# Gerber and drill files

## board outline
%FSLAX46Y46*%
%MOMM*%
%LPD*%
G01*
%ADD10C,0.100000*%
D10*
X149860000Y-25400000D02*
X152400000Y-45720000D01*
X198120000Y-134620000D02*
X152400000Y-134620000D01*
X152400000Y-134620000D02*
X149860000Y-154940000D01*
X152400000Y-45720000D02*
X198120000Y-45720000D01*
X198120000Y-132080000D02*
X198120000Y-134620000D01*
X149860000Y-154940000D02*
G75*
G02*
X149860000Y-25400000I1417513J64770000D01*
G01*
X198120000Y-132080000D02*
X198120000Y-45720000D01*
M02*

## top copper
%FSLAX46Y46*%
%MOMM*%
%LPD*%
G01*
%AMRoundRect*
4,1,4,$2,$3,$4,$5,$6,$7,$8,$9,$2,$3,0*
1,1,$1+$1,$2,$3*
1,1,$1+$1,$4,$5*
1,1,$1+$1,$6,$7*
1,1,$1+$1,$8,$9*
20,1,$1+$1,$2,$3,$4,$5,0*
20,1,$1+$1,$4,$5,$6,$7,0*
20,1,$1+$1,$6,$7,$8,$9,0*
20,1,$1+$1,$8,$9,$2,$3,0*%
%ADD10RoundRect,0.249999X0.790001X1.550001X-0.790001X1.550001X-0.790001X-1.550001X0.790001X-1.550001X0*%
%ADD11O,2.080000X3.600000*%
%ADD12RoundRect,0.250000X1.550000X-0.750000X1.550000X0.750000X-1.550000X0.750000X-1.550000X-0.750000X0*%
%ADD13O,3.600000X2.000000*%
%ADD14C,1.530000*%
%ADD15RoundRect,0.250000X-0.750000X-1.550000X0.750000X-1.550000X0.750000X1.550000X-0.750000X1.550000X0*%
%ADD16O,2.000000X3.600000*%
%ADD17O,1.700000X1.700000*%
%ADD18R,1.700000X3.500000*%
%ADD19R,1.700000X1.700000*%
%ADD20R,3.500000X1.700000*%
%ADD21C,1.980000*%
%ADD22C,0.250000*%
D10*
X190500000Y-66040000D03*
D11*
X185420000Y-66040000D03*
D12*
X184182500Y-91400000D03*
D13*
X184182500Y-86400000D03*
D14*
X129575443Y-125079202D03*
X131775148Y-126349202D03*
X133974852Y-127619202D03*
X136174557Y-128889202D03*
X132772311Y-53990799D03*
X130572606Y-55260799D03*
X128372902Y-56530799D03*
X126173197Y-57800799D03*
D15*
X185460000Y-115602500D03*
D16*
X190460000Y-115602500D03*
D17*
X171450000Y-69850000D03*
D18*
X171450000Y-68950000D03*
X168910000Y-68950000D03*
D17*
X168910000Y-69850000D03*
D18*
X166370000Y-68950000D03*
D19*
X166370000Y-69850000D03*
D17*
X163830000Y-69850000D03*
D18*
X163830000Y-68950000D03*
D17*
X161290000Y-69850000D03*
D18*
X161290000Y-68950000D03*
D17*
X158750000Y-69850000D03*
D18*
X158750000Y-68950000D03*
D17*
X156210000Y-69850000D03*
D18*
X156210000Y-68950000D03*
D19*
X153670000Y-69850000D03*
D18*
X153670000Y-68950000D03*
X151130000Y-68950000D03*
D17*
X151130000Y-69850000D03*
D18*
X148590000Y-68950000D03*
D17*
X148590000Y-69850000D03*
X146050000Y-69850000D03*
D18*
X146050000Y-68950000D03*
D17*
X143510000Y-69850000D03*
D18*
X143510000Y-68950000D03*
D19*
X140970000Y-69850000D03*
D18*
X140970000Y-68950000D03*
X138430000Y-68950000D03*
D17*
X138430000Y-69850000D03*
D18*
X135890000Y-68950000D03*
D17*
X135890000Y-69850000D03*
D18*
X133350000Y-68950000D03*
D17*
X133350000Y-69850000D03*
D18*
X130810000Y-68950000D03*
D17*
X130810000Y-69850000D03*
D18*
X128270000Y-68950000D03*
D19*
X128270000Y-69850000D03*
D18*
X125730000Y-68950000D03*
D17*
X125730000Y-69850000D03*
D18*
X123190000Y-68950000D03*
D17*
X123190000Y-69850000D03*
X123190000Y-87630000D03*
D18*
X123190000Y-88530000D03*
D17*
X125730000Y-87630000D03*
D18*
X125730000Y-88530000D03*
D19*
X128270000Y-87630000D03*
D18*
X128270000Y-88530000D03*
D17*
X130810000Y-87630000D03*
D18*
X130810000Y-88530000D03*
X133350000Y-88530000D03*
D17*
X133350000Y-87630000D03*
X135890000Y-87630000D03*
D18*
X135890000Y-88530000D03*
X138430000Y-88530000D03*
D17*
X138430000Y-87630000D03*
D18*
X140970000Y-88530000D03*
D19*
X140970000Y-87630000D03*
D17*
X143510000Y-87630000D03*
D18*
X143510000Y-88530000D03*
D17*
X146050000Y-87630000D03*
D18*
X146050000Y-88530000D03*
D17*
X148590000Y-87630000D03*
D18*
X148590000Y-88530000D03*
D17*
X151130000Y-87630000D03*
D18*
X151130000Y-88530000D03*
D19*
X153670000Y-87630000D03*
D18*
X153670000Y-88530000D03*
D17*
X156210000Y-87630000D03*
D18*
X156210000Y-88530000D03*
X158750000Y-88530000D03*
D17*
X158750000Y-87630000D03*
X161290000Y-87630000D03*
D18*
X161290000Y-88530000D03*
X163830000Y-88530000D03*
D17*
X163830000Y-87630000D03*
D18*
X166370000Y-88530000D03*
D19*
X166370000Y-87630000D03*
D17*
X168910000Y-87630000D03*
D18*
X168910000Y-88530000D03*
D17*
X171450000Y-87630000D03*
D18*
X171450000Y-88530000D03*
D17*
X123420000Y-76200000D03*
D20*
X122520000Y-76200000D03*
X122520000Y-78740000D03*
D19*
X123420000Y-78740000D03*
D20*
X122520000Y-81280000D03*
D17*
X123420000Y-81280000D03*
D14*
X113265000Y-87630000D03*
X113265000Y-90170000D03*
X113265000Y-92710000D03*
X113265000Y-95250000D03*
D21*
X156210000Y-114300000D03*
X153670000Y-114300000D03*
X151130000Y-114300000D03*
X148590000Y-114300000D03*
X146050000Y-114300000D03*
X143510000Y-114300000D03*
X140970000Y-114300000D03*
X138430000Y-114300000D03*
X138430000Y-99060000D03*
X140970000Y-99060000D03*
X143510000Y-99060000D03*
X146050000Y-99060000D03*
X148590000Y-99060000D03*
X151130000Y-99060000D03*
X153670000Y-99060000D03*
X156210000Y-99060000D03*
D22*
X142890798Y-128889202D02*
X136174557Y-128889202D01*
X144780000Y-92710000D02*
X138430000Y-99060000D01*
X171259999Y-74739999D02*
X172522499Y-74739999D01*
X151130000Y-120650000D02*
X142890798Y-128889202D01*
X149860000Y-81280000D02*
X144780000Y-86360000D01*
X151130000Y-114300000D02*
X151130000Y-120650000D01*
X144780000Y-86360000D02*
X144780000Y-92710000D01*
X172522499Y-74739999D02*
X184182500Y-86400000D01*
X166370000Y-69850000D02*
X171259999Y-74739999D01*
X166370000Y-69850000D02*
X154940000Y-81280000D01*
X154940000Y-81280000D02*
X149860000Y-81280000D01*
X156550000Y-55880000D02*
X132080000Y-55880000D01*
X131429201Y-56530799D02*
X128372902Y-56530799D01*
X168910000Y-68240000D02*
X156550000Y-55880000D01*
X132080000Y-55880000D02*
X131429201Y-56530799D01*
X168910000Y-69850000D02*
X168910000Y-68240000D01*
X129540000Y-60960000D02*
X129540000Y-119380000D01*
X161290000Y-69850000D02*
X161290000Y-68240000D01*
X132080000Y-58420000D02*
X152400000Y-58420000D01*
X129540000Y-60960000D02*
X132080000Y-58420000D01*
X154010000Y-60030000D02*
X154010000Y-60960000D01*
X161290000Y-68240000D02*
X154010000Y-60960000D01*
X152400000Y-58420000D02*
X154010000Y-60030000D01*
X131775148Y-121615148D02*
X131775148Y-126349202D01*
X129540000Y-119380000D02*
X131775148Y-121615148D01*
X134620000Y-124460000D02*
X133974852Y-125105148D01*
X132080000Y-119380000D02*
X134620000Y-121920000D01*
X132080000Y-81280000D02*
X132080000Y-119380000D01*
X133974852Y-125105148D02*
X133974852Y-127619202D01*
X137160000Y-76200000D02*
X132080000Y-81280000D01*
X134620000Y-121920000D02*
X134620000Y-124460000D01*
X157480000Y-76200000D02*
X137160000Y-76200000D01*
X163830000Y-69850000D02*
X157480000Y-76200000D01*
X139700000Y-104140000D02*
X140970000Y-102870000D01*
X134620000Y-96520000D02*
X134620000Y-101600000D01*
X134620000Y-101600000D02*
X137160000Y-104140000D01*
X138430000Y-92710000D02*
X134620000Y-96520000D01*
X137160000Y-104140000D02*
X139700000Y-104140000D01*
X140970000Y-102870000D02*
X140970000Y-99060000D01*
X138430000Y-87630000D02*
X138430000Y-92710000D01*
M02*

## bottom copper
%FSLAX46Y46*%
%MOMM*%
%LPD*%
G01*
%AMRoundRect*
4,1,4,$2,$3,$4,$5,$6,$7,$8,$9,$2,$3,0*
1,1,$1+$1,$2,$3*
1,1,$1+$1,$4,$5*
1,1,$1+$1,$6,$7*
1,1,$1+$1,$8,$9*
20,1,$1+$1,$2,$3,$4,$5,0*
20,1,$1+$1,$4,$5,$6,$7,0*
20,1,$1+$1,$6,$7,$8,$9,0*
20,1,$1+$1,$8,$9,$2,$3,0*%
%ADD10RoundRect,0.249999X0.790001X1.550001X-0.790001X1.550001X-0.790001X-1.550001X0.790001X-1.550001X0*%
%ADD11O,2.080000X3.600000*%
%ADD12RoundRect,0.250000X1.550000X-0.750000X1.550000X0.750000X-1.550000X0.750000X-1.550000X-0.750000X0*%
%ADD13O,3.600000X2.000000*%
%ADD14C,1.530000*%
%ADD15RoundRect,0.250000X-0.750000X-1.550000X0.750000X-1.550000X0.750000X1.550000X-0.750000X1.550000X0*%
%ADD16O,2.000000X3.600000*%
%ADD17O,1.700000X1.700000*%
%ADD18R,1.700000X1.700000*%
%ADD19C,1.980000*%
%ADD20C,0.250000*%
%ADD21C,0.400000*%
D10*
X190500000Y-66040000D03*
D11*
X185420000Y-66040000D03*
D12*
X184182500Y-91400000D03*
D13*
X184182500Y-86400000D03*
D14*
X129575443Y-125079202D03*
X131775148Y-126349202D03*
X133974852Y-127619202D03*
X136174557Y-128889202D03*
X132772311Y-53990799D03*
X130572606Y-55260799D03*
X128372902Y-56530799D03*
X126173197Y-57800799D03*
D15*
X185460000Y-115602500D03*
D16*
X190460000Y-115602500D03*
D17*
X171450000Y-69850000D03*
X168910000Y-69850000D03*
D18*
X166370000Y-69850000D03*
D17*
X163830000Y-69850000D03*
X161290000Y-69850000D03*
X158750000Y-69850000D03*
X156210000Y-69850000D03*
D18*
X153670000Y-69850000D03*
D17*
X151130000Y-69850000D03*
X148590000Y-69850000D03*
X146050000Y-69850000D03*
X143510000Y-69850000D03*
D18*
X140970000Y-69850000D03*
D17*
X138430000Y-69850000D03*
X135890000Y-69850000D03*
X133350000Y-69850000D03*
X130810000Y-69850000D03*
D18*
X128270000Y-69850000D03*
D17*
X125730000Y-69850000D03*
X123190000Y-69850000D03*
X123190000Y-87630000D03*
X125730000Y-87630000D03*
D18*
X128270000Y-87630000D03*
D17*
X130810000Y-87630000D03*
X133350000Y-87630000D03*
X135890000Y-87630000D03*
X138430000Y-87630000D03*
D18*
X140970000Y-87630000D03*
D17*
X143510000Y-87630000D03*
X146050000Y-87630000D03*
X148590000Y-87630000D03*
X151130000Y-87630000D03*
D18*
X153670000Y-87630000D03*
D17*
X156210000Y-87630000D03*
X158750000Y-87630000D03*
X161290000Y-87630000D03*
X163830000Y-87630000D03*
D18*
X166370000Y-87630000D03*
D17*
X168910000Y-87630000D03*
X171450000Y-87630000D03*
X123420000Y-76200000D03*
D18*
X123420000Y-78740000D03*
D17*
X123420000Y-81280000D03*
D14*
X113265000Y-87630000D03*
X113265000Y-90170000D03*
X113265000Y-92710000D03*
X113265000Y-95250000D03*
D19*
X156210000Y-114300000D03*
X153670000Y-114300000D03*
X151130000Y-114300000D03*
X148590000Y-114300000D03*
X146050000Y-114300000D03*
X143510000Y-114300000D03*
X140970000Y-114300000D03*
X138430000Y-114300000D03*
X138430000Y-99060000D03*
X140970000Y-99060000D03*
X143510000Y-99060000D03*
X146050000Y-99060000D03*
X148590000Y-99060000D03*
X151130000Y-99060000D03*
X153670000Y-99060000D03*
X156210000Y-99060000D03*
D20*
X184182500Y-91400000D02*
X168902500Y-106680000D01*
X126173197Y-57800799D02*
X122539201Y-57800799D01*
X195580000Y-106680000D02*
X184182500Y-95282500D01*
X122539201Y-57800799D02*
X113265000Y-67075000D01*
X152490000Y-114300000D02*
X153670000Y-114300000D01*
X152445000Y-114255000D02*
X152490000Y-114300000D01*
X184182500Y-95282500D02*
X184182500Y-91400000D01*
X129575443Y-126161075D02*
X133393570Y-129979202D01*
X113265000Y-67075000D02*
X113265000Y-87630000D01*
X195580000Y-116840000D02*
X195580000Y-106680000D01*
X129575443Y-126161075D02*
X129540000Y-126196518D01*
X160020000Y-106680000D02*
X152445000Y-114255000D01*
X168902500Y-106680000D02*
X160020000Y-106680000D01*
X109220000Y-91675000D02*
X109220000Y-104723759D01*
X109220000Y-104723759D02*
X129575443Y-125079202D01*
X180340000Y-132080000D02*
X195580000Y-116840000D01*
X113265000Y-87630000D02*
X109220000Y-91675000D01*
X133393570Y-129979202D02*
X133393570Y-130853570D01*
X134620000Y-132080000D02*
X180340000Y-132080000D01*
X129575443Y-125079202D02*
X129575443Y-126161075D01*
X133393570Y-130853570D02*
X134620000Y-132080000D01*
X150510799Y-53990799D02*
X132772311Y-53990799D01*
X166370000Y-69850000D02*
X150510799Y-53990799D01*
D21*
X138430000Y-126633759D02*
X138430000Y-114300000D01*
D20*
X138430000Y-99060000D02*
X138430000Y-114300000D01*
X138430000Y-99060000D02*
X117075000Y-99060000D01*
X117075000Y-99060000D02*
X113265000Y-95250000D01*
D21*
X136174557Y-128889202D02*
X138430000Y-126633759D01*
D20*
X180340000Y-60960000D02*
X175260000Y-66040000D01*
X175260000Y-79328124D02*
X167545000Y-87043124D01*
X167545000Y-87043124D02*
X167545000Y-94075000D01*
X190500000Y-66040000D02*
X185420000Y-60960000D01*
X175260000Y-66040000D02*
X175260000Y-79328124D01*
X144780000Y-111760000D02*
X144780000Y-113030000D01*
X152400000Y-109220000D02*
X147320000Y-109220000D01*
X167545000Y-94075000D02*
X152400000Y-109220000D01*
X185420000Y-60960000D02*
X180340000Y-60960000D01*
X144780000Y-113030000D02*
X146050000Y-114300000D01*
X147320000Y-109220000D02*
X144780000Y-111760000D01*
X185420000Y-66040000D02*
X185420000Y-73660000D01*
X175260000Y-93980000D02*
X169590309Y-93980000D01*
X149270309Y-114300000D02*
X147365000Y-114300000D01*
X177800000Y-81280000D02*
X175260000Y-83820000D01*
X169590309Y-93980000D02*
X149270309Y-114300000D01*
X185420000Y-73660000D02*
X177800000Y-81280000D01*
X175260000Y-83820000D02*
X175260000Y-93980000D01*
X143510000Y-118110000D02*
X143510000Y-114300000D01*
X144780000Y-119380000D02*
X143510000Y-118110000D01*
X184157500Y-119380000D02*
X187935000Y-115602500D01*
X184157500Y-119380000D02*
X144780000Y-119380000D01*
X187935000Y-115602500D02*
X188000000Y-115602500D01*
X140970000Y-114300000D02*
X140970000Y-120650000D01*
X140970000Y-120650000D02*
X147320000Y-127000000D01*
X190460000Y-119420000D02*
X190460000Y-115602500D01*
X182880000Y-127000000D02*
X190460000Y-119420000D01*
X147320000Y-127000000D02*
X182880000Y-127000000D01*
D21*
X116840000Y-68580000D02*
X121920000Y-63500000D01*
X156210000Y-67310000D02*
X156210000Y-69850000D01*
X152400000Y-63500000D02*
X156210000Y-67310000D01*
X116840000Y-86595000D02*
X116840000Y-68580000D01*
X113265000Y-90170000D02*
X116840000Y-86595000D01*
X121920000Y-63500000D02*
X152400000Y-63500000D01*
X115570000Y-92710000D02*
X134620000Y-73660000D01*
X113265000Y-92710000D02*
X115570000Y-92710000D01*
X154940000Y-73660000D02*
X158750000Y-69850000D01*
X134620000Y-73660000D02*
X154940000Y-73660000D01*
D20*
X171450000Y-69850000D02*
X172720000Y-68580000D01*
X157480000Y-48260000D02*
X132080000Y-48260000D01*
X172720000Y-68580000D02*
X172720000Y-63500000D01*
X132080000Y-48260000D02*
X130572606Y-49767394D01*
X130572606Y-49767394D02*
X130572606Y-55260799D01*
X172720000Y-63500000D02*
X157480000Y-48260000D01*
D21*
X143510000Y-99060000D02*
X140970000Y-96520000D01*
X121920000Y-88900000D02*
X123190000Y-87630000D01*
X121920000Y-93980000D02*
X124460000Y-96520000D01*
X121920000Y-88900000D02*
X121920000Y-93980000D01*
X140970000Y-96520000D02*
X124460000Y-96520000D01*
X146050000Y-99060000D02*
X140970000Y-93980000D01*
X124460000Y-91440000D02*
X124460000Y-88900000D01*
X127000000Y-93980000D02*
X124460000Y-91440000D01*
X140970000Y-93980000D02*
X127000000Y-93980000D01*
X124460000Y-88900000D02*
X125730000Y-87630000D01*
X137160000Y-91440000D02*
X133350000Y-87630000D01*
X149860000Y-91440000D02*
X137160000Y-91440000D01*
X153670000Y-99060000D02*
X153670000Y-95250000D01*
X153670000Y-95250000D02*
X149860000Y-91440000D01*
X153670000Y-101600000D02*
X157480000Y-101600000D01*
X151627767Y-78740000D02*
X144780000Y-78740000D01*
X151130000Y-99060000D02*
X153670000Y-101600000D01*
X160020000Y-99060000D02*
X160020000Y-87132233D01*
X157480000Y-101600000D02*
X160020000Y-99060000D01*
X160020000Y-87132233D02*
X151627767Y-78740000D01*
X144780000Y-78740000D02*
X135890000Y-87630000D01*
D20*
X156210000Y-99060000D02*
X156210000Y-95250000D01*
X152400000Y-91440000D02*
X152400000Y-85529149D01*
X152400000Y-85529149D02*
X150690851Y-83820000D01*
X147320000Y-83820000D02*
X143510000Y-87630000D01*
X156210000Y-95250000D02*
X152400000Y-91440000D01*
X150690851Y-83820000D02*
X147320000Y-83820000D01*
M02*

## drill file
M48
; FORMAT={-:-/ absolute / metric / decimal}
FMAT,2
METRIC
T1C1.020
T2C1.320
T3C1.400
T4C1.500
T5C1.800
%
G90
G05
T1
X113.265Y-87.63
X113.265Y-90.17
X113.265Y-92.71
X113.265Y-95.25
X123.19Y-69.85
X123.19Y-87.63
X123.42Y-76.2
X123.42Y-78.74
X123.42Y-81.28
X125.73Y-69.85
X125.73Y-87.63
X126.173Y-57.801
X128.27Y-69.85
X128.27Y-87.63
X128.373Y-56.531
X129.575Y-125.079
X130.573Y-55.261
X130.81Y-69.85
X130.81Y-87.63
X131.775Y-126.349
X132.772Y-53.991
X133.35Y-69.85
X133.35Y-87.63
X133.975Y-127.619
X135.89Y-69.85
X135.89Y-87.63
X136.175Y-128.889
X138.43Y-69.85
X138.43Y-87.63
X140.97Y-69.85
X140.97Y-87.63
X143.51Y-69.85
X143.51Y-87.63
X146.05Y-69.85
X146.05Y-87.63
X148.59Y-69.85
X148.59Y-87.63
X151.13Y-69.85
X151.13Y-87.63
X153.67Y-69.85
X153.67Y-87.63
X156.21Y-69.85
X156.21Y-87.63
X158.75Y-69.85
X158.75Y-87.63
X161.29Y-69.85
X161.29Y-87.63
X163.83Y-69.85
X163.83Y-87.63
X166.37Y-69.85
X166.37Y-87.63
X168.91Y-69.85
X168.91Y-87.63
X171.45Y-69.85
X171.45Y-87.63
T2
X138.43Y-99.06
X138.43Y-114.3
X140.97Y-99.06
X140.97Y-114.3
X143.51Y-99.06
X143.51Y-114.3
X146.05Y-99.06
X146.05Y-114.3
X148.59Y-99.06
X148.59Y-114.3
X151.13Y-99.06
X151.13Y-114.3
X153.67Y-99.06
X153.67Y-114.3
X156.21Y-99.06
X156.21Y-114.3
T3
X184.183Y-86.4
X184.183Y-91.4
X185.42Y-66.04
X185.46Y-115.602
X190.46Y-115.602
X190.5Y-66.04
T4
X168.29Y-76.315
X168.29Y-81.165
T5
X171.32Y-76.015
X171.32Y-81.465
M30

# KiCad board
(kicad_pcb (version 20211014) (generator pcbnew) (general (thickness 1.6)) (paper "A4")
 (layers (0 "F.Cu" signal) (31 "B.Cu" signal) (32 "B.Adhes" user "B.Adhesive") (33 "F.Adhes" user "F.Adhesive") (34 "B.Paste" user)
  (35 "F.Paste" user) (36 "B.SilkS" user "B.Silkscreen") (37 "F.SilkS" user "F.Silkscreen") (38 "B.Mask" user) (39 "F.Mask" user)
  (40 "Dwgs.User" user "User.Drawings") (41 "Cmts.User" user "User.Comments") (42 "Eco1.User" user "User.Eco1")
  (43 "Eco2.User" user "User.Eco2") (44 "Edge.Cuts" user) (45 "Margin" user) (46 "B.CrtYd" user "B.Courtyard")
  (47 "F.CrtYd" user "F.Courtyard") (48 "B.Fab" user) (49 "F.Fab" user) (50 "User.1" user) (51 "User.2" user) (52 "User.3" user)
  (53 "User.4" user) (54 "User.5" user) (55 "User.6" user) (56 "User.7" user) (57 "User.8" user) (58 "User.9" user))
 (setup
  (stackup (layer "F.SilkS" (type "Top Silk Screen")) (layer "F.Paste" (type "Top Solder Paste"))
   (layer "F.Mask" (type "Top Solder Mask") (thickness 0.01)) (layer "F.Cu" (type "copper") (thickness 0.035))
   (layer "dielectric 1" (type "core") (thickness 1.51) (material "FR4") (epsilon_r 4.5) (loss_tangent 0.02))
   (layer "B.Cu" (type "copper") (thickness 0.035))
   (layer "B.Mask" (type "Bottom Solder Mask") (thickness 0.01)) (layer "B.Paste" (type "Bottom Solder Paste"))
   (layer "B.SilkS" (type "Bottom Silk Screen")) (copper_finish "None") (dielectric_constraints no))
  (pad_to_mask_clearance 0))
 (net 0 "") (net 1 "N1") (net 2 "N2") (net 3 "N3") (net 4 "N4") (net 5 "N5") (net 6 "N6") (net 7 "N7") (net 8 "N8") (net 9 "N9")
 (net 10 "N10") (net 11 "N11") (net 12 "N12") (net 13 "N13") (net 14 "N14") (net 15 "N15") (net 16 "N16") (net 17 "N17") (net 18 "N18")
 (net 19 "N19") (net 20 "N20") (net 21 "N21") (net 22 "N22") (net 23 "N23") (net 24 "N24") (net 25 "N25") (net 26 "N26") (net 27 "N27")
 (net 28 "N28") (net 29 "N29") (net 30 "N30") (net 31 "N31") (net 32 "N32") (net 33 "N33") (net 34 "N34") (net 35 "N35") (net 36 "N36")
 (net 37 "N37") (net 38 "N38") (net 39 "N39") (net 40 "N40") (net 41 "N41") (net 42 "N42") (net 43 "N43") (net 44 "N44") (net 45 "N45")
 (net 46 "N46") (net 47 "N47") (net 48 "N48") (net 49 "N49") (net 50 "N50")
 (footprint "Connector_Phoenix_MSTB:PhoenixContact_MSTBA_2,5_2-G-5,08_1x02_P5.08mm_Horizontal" (layer "F.Cu") (at 190.5 66.04 180)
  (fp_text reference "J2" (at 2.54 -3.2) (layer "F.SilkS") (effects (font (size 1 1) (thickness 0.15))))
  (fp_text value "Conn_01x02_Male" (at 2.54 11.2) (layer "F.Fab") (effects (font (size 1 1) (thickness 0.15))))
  (pad "1" thru_hole roundrect (at 0 0 180) (size 2.08 3.6) (drill 1.4) (layers *.Cu *.Mask) (roundrect_rratio 0.120192) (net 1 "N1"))
  (pad "2" thru_hole oval (at 5.08 0 180) (size 2.08 3.6) (drill 1.4) (layers *.Cu *.Mask) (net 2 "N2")))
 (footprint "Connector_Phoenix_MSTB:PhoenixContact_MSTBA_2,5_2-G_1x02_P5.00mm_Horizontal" (layer "F.Cu") (at 184.1825 91.4 90)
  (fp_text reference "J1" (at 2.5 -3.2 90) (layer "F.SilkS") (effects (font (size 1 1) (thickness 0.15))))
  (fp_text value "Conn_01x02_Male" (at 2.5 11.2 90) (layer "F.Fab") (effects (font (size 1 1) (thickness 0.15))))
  (pad "1" thru_hole roundrect (at 0 0 90) (size 2 3.6) (drill 1.4) (layers *.Cu *.Mask) (roundrect_rratio 0.125) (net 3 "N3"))
  (pad "2" thru_hole oval (at 5 0 90) (size 2 3.6) (drill 1.4) (layers *.Cu *.Mask) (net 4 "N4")))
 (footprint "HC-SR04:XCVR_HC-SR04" (layer "F.Cu") (at 132.875 126.984202 -30)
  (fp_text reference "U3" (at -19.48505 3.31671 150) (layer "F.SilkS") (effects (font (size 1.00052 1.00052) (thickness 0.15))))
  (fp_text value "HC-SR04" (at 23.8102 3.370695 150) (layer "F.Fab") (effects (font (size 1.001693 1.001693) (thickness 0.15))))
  (pad "1" thru_hole circle locked (at -3.81 0 330) (size 1.53 1.53) (drill 1.02) (layers *.Cu *.Mask) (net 3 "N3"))
  (pad "2" thru_hole circle locked (at -1.27 0 330) (size 1.53 1.53) (drill 1.02) (layers *.Cu *.Mask) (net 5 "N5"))
  (pad "3" thru_hole circle locked (at 1.27 0 330) (size 1.53 1.53) (drill 1.02) (layers *.Cu *.Mask) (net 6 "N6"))
  (pad "4" thru_hole circle locked (at 3.81 0 330) (size 1.53 1.53) (drill 1.02) (layers *.Cu *.Mask) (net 4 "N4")))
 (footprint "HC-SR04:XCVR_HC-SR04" (layer "F.Cu") (at 129.472754 55.895799 -150)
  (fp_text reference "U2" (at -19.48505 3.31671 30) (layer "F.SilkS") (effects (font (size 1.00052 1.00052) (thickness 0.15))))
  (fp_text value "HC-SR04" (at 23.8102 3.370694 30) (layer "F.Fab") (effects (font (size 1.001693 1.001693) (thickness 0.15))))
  (pad "1" thru_hole circle locked (at -3.81 0 210) (size 1.53 1.53) (drill 1.02) (layers *.Cu *.Mask) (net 3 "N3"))
  (pad "2" thru_hole circle locked (at -1.27 0 210) (size 1.53 1.53) (drill 1.02) (layers *.Cu *.Mask) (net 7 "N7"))
  (pad "3" thru_hole circle locked (at 1.27 0 210) (size 1.53 1.53) (drill 1.02) (layers *.Cu *.Mask) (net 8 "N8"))
  (pad "4" thru_hole circle locked (at 3.81 0 210) (size 1.53 1.53) (drill 1.02) (layers *.Cu *.Mask) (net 4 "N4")))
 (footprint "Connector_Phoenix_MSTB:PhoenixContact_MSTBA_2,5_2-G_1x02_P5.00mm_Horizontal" (layer "F.Cu") (at 185.46 115.6025)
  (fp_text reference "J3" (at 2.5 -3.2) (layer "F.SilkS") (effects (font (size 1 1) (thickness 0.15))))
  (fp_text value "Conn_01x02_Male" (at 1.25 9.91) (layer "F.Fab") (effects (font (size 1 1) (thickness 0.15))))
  (pad "1" thru_hole roundrect (at 0 0) (size 2 3.6) (drill 1.4) (layers *.Cu *.Mask) (roundrect_rratio 0.125) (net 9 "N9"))
  (pad "2" thru_hole oval (at 5 0) (size 2 3.6) (drill 1.4) (layers *.Cu *.Mask) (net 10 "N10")))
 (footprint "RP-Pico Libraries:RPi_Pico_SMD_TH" (layer "F.Cu") (at 147.32 78.74 -90)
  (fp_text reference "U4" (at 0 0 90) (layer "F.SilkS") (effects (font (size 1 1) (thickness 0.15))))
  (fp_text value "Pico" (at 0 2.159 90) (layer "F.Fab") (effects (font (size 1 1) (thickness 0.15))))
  (pad "" np_thru_hole oval (at -2.725 -24 270) (size 1.8 1.8) (drill 1.8) (layers *.Cu *.Mask))
  (pad "" np_thru_hole oval (at -2.425 -20.97 270) (size 1.5 1.5) (drill 1.5) (layers *.Cu *.Mask))
  (pad "" np_thru_hole oval (at 2.425 -20.97 270) (size 1.5 1.5) (drill 1.5) (layers *.Cu *.Mask))
  (pad "" np_thru_hole oval (at 2.725 -24 270) (size 1.8 1.8) (drill 1.8) (layers *.Cu *.Mask))
  (pad "1" thru_hole oval (at -8.89 -24.13 270) (size 1.7 1.7) (drill 1.02) (layers *.Cu *.Mask) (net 8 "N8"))
  (pad "1" smd rect (at -8.89 -24.13 270) (size 3.5 1.7) (drill (offset -0.9 0)) (layers "F.Cu" "F.Mask") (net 8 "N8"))
  (pad "2" smd rect (at -8.89 -21.59 270) (size 3.5 1.7) (drill (offset -0.9 0)) (layers "F.Cu" "F.Mask") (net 7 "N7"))
  (pad "2" thru_hole oval (at -8.89 -21.59 270) (size 1.7 1.7) (drill 1.02) (layers *.Cu *.Mask) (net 7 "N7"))
  (pad "3" smd rect (at -8.89 -19.05 270) (size 3.5 1.7) (drill (offset -0.9 0)) (layers "F.Cu" "F.Mask") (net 4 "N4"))
  (pad "3" thru_hole rect (at -8.89 -19.05 270) (size 1.7 1.7) (drill 1.02) (layers *.Cu *.Mask) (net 4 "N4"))
  (pad "4" thru_hole oval (at -8.89 -16.51 270) (size 1.7 1.7) (drill 1.02) (layers *.Cu *.Mask) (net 6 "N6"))
  (pad "4" smd rect (at -8.89 -16.51 270) (size 3.5 1.7) (drill (offset -0.9 0)) (layers "F.Cu" "F.Mask") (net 6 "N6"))
  (pad "5" thru_hole oval (at -8.89 -13.97 270) (size 1.7 1.7) (drill 1.02) (layers *.Cu *.Mask) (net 5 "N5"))
  (pad "5" smd rect (at -8.89 -13.97 270) (size 3.5 1.7) (drill (offset -0.9 0)) (layers "F.Cu" "F.Mask") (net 5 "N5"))
  (pad "6" thru_hole oval (at -8.89 -11.43 270) (size 1.7 1.7) (drill 1.02) (layers *.Cu *.Mask) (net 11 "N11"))
  (pad "6" smd rect (at -8.89 -11.43 270) (size 3.5 1.7) (drill (offset -0.9 0)) (layers "F.Cu" "F.Mask") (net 11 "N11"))
  (pad "7" thru_hole oval (at -8.89 -8.89 270) (size 1.7 1.7) (drill 1.02) (layers *.Cu *.Mask) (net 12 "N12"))
  (pad "7" smd rect (at -8.89 -8.89 270) (size 3.5 1.7) (drill (offset -0.9 0)) (layers "F.Cu" "F.Mask") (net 12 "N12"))
  (pad "8" thru_hole rect (at -8.89 -6.35 270) (size 1.7 1.7) (drill 1.02) (layers *.Cu *.Mask) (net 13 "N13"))
  (pad "8" smd rect (at -8.89 -6.35 270) (size 3.5 1.7) (drill (offset -0.9 0)) (layers "F.Cu" "F.Mask") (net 13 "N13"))
  (pad "9" smd rect (at -8.89 -3.81 270) (size 3.5 1.7) (drill (offset -0.9 0)) (layers "F.Cu" "F.Mask") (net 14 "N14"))
  (pad "9" thru_hole oval (at -8.89 -3.81 270) (size 1.7 1.7) (drill 1.02) (layers *.Cu *.Mask) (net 14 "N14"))
  (pad "10" smd rect (at -8.89 -1.27 270) (size 3.5 1.7) (drill (offset -0.9 0)) (layers "F.Cu" "F.Mask") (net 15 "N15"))
  (pad "10" thru_hole oval (at -8.89 -1.27 270) (size 1.7 1.7) (drill 1.02) (layers *.Cu *.Mask) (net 15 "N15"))
  (pad "11" thru_hole oval (at -8.89 1.27 270) (size 1.7 1.7) (drill 1.02) (layers *.Cu *.Mask) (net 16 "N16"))
  (pad "11" smd rect (at -8.89 1.27 270) (size 3.5 1.7) (drill (offset -0.9 0)) (layers "F.Cu" "F.Mask") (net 16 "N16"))
  (pad "12" thru_hole oval (at -8.89 3.81 270) (size 1.7 1.7) (drill 1.02) (layers *.Cu *.Mask) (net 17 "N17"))
  (pad "12" smd rect (at -8.89 3.81 270) (size 3.5 1.7) (drill (offset -0.9 0)) (layers "F.Cu" "F.Mask") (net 17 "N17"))
  (pad "13" thru_hole rect (at -8.89 6.35 270) (size 1.7 1.7) (drill 1.02) (layers *.Cu *.Mask) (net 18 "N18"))
  (pad "13" smd rect (at -8.89 6.35 270) (size 3.5 1.7) (drill (offset -0.9 0)) (layers "F.Cu" "F.Mask") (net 18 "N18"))
  (pad "14" smd rect (at -8.89 8.89 270) (size 3.5 1.7) (drill (offset -0.9 0)) (layers "F.Cu" "F.Mask") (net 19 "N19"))
  (pad "14" thru_hole oval (at -8.89 8.89 270) (size 1.7 1.7) (drill 1.02) (layers *.Cu *.Mask) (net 19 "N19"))
  (pad "15" smd rect (at -8.89 11.43 270) (size 3.5 1.7) (drill (offset -0.9 0)) (layers "F.Cu" "F.Mask") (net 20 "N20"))
  (pad "15" thru_hole oval (at -8.89 11.43 270) (size 1.7 1.7) (drill 1.02) (layers *.Cu *.Mask) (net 20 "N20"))
  (pad "16" smd rect (at -8.89 13.97 270) (size 3.5 1.7) (drill (offset -0.9 0)) (layers "F.Cu" "F.Mask") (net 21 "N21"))
  (pad "16" thru_hole oval (at -8.89 13.97 270) (size 1.7 1.7) (drill 1.02) (layers *.Cu *.Mask) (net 21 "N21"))
  (pad "17" smd rect (at -8.89 16.51 270) (size 3.5 1.7) (drill (offset -0.9 0)) (layers "F.Cu" "F.Mask") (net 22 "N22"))
  (pad "17" thru_hole oval (at -8.89 16.51 270) (size 1.7 1.7) (drill 1.02) (layers *.Cu *.Mask) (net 22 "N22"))
  (pad "18" smd rect (at -8.89 19.05 270) (size 3.5 1.7) (drill (offset -0.9 0)) (layers "F.Cu" "F.Mask") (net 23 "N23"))
  (pad "18" thru_hole rect (at -8.89 19.05 270) (size 1.7 1.7) (drill 1.02) (layers *.Cu *.Mask) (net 23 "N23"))
  (pad "19" smd rect (at -8.89 21.59 270) (size 3.5 1.7) (drill (offset -0.9 0)) (layers "F.Cu" "F.Mask") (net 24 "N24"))
  (pad "19" thru_hole oval (at -8.89 21.59 270) (size 1.7 1.7) (drill 1.02) (layers *.Cu *.Mask) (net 24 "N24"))
  (pad "20" smd rect (at -8.89 24.13 270) (size 3.5 1.7) (drill (offset -0.9 0)) (layers "F.Cu" "F.Mask") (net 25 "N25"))
  (pad "20" thru_hole oval (at -8.89 24.13 270) (size 1.7 1.7) (drill 1.02) (layers *.Cu *.Mask) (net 25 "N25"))
  (pad "21" thru_hole oval (at 8.89 24.13 270) (size 1.7 1.7) (drill 1.02) (layers *.Cu *.Mask) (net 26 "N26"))
  (pad "21" smd rect (at 8.89 24.13 270) (size 3.5 1.7) (drill (offset 0.9 0)) (layers "F.Cu" "F.Mask") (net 26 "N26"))
  (pad "22" thru_hole oval (at 8.89 21.59 270) (size 1.7 1.7) (drill 1.02) (layers *.Cu *.Mask) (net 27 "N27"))
  (pad "22" smd rect (at 8.89 21.59 270) (size 3.5 1.7) (drill (offset 0.9 0)) (layers "F.Cu" "F.Mask") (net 27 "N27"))
  (pad "23" thru_hole rect (at 8.89 19.05 270) (size 1.7 1.7) (drill 1.02) (layers *.Cu *.Mask) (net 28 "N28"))
  (pad "23" smd rect (at 8.89 19.05 270) (size 3.5 1.7) (drill (offset 0.9 0)) (layers "F.Cu" "F.Mask") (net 28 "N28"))
  (pad "24" thru_hole oval (at 8.89 16.51 270) (size 1.7 1.7) (drill 1.02) (layers *.Cu *.Mask) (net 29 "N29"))
  (pad "24" smd rect (at 8.89 16.51 270) (size 3.5 1.7) (drill (offset 0.9 0)) (layers "F.Cu" "F.Mask") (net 29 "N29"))
  (pad "25" smd rect (at 8.89 13.97 270) (size 3.5 1.7) (drill (offset 0.9 0)) (layers "F.Cu" "F.Mask") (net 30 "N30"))
  (pad "25" thru_hole oval (at 8.89 13.97 270) (size 1.7 1.7) (drill 1.02) (layers *.Cu *.Mask) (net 30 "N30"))
  (pad "26" thru_hole oval (at 8.89 11.43 270) (size 1.7 1.7) (drill 1.02) (layers *.Cu *.Mask) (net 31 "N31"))
  (pad "26" smd rect (at 8.89 11.43 270) (size 3.5 1.7) (drill (offset 0.9 0)) (layers "F.Cu" "F.Mask") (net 31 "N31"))
  (pad "27" smd rect (at 8.89 8.89 270) (size 3.5 1.7) (drill (offset 0.9 0)) (layers "F.Cu" "F.Mask") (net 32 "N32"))
  (pad "27" thru_hole oval (at 8.89 8.89 270) (size 1.7 1.7) (drill 1.02) (layers *.Cu *.Mask) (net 32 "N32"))
  (pad "28" smd rect (at 8.89 6.35 270) (size 3.5 1.7) (drill (offset 0.9 0)) (layers "F.Cu" "F.Mask") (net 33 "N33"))
  (pad "28" thru_hole rect (at 8.89 6.35 270) (size 1.7 1.7) (drill 1.02) (layers *.Cu *.Mask) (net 33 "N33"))
  (pad "29" thru_hole oval (at 8.89 3.81 270) (size 1.7 1.7) (drill 1.02) (layers *.Cu *.Mask) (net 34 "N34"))
  (pad "29" smd rect (at 8.89 3.81 270) (size 3.5 1.7) (drill (offset 0.9 0)) (layers "F.Cu" "F.Mask") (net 34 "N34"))
  (pad "30" thru_hole oval (at 8.89 1.27 270) (size 1.7 1.7) (drill 1.02) (layers *.Cu *.Mask) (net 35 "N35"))
  (pad "30" smd rect (at 8.89 1.27 270) (size 3.5 1.7) (drill (offset 0.9 0)) (layers "F.Cu" "F.Mask") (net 35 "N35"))
  (pad "31" thru_hole oval (at 8.89 -1.27 270) (size 1.7 1.7) (drill 1.02) (layers *.Cu *.Mask) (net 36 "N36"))
  (pad "31" smd rect (at 8.89 -1.27 270) (size 3.5 1.7) (drill (offset 0.9 0)) (layers "F.Cu" "F.Mask") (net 36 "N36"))
  (pad "32" thru_hole oval (at 8.89 -3.81 270) (size 1.7 1.7) (drill 1.02) (layers *.Cu *.Mask) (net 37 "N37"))
  (pad "32" smd rect (at 8.89 -3.81 270) (size 3.5 1.7) (drill (offset 0.9 0)) (layers "F.Cu" "F.Mask") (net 37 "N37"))
  (pad "33" thru_hole rect (at 8.89 -6.35 270) (size 1.7 1.7) (drill 1.02) (layers *.Cu *.Mask) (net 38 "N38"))
  (pad "33" smd rect (at 8.89 -6.35 270) (size 3.5 1.7) (drill (offset 0.9 0)) (layers "F.Cu" "F.Mask") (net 38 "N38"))
  (pad "34" thru_hole oval (at 8.89 -8.89 270) (size 1.7 1.7) (drill 1.02) (layers *.Cu *.Mask) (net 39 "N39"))
  (pad "34" smd rect (at 8.89 -8.89 270) (size 3.5 1.7) (drill (offset 0.9 0)) (layers "F.Cu" "F.Mask") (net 39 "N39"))
  (pad "35" smd rect (at 8.89 -11.43 270) (size 3.5 1.7) (drill (offset 0.9 0)) (layers "F.Cu" "F.Mask") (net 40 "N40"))
  (pad "35" thru_hole oval (at 8.89 -11.43 270) (size 1.7 1.7) (drill 1.02) (layers *.Cu *.Mask) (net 40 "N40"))
  (pad "36" thru_hole oval (at 8.89 -13.97 270) (size 1.7 1.7) (drill 1.02) (layers *.Cu *.Mask) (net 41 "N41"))
  (pad "36" smd rect (at 8.89 -13.97 270) (size 3.5 1.7) (drill (offset 0.9 0)) (layers "F.Cu" "F.Mask") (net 41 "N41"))
  (pad "37" smd rect (at 8.89 -16.51 270) (size 3.5 1.7) (drill (offset 0.9 0)) (layers "F.Cu" "F.Mask") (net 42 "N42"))
  (pad "37" thru_hole oval (at 8.89 -16.51 270) (size 1.7 1.7) (drill 1.02) (layers *.Cu *.Mask) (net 42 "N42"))
  (pad "38" smd rect (at 8.89 -19.05 270) (size 3.5 1.7) (drill (offset 0.9 0)) (layers "F.Cu" "F.Mask") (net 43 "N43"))
  (pad "38" thru_hole rect (at 8.89 -19.05 270) (size 1.7 1.7) (drill 1.02) (layers *.Cu *.Mask) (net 43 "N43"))
  (pad "39" thru_hole oval (at 8.89 -21.59 270) (size 1.7 1.7) (drill 1.02) (layers *.Cu *.Mask) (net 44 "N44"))
  (pad "39" smd rect (at 8.89 -21.59 270) (size 3.5 1.7) (drill (offset 0.9 0)) (layers "F.Cu" "F.Mask") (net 44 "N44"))
  (pad "40" thru_hole oval (at 8.89 -24.13 270) (size 1.7 1.7) (drill 1.02) (layers *.Cu *.Mask) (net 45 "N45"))
  (pad "40" smd rect (at 8.89 -24.13 270) (size 3.5 1.7) (drill (offset 0.9 0)) (layers "F.Cu" "F.Mask") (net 45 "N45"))
  (pad "41" thru_hole oval (at -2.54 23.9 270) (size 1.7 1.7) (drill 1.02) (layers *.Cu *.Mask) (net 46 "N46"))
  (pad "41" smd rect (at -2.54 23.9) (size 3.5 1.7) (drill (offset -0.9 0)) (layers "F.Cu" "F.Mask") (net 46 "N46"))
  (pad "42" smd rect (at 0 23.9) (size 3.5 1.7) (drill (offset -0.9 0)) (layers "F.Cu" "F.Mask") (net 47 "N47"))
  (pad "42" thru_hole rect (at 0 23.9 270) (size 1.7 1.7) (drill 1.02) (layers *.Cu *.Mask) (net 47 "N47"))
  (pad "43" smd rect (at 2.54 23.9) (size 3.5 1.7) (drill (offset -0.9 0)) (layers "F.Cu" "F.Mask") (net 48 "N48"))
  (pad "43" thru_hole oval (at 2.54 23.9 270) (size 1.7 1.7) (drill 1.02) (layers *.Cu *.Mask) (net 48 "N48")))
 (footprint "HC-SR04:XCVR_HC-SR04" (layer "F.Cu") (at 113.265 91.44 -90)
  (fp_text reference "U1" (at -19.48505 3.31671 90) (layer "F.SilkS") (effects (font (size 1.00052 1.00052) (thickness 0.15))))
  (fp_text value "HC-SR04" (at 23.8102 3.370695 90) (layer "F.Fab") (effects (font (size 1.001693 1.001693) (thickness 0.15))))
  (pad "1" thru_hole circle locked (at -3.81 0 270) (size 1.53 1.53) (drill 1.02) (layers *.Cu *.Mask) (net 3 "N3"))
  (pad "2" thru_hole circle locked (at -1.27 0 270) (size 1.53 1.53) (drill 1.02) (layers *.Cu *.Mask) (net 12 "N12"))
  (pad "3" thru_hole circle locked (at 1.27 0 270) (size 1.53 1.53) (drill 1.02) (layers *.Cu *.Mask) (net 11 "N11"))
  (pad "4" thru_hole circle locked (at 3.81 0 270) (size 1.53 1.53) (drill 1.02) (layers *.Cu *.Mask) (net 4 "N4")))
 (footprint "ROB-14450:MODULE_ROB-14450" (layer "B.Cu") (at 147.32 106.68 90)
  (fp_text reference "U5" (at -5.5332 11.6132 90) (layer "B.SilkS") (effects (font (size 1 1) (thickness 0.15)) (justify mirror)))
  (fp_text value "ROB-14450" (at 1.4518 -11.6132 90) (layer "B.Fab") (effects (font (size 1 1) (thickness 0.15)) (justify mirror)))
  (pad "1" thru_hole circle locked (at -7.62 8.89 90) (size 1.98 1.98) (drill 1.32) (layers *.Cu *.Mask) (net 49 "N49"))
  (pad "2" thru_hole circle locked (at -7.62 6.35 90) (size 1.98 1.98) (drill 1.32) (layers *.Cu *.Mask) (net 3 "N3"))
  (pad "3" thru_hole circle locked (at -7.62 3.81 90) (size 1.98 1.98) (drill 1.32) (layers *.Cu *.Mask) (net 4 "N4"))
  (pad "4" thru_hole circle locked (at -7.62 1.27 90) (size 1.98 1.98) (drill 1.32) (layers *.Cu *.Mask) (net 2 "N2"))
  (pad "5" thru_hole circle locked (at -7.62 -1.27 90) (size 1.98 1.98) (drill 1.32) (layers *.Cu *.Mask) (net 1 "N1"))
  (pad "6" thru_hole circle locked (at -7.62 -3.81 90) (size 1.98 1.98) (drill 1.32) (layers *.Cu *.Mask) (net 9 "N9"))
  (pad "7" thru_hole circle locked (at -7.62 -6.35 90) (size 1.98 1.98) (drill 1.32) (layers *.Cu *.Mask) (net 10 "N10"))
  (pad "8" thru_hole circle locked (at -7.62 -8.89 90) (size 1.98 1.98) (drill 1.32) (layers *.Cu *.Mask) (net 4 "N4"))
  (pad "9" thru_hole circle locked (at 7.62 -8.89 90) (size 1.98 1.98) (drill 1.32) (layers *.Cu *.Mask) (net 4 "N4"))
  (pad "10" thru_hole circle locked (at 7.62 -6.35 90) (size 1.98 1.98) (drill 1.32) (layers *.Cu *.Mask) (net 32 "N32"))
  (pad "11" thru_hole circle locked (at 7.62 -3.81 90) (size 1.98 1.98) (drill 1.32) (layers *.Cu *.Mask) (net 26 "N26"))
  (pad "12" thru_hole circle locked (at 7.62 -1.27 90) (size 1.98 1.98) (drill 1.32) (layers *.Cu *.Mask) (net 27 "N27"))
  (pad "13" thru_hole circle locked (at 7.62 1.27 90) (size 1.98 1.98) (drill 1.32) (layers *.Cu *.Mask) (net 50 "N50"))
  (pad "14" thru_hole circle locked (at 7.62 3.81 90) (size 1.98 1.98) (drill 1.32) (layers *.Cu *.Mask) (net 31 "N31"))
  (pad "15" thru_hole circle locked (at 7.62 6.35 90) (size 1.98 1.98) (drill 1.32) (layers *.Cu *.Mask) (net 30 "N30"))
  (pad "16" thru_hole circle locked (at 7.62 8.89 90) (size 1.98 1.98) (drill 1.32) (layers *.Cu *.Mask) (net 34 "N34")))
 (gr_line (start 149.86 25.4) (end 152.4 45.72) (layer "Edge.Cuts") (width 0.1))
 (gr_line (start 198.12 134.62) (end 152.4 134.62) (layer "Edge.Cuts") (width 0.1))
 (gr_line (start 152.4 134.62) (end 149.86 154.94) (layer "Edge.Cuts") (width 0.1))
 (gr_line (start 152.4 45.72) (end 198.12 45.72) (layer "Edge.Cuts") (width 0.1))
 (gr_line (start 198.12 132.08) (end 198.12 134.62) (layer "Edge.Cuts") (width 0.1))
 (gr_arc (start 149.86 154.94) (mid 86.492003 90.17) (end 149.86 25.4) (layer "Edge.Cuts") (width 0.1))
 (gr_line (start 198.12 132.08) (end 198.12 45.72) (layer "Edge.Cuts") (width 0.1))
 (segment (start 184.1825 91.4) (end 168.9025 106.68) (width 0.25) (layer "B.Cu") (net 3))
 (segment (start 126.173197 57.800799) (end 122.539201 57.800799) (width 0.25) (layer "B.Cu") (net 3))
 (segment (start 195.58 106.68) (end 184.1825 95.2825) (width 0.25) (layer "B.Cu") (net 3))
 (segment (start 122.539201 57.800799) (end 113.265 67.075) (width 0.25) (layer "B.Cu") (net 3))
 (segment (start 152.49 114.3) (end 153.67 114.3) (width 0.25) (layer "B.Cu") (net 3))
 (segment (start 152.445 114.255) (end 152.49 114.3) (width 0.25) (layer "B.Cu") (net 3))
 (segment (start 184.1825 95.2825) (end 184.1825 91.4) (width 0.25) (layer "B.Cu") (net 3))
 (segment (start 129.575443 126.161075) (end 133.39357 129.979202) (width 0.25) (layer "B.Cu") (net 3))
 (segment (start 113.265 67.075) (end 113.265 87.63) (width 0.25) (layer "B.Cu") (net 3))
 (segment (start 195.58 116.84) (end 195.58 106.68) (width 0.25) (layer "B.Cu") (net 3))
 (segment (start 129.575443 126.161075) (end 129.54 126.196518) (width 0.25) (layer "B.Cu") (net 3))
 (segment (start 160.02 106.68) (end 152.445 114.255) (width 0.25) (layer "B.Cu") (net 3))
 (segment (start 168.9025 106.68) (end 160.02 106.68) (width 0.25) (layer "B.Cu") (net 3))
 (segment (start 109.22 91.675) (end 109.22 104.723759) (width 0.25) (layer "B.Cu") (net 3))
 (segment (start 109.22 104.723759) (end 129.575443 125.079202) (width 0.25) (layer "B.Cu") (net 3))
 (segment (start 180.34 132.08) (end 195.58 116.84) (width 0.25) (layer "B.Cu") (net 3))
 (segment (start 113.265 87.63) (end 109.22 91.675) (width 0.25) (layer "B.Cu") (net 3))
 (segment (start 133.39357 129.979202) (end 133.39357 130.85357) (width 0.25) (layer "B.Cu") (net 3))
 (segment (start 134.62 132.08) (end 180.34 132.08) (width 0.25) (layer "B.Cu") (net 3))
 (segment (start 129.575443 125.079202) (end 129.575443 126.161075) (width 0.25) (layer "B.Cu") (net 3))
 (segment (start 133.39357 130.85357) (end 134.62 132.08) (width 0.25) (layer "B.Cu") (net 3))
 (segment (start 142.890798 128.889202) (end 136.174557 128.889202) (width 0.25) (layer "F.Cu") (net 4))
 (segment (start 144.78 92.71) (end 138.43 99.06) (width 0.25) (layer "F.Cu") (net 4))
 (segment (start 171.259999 74.739999) (end 172.522499 74.739999) (width 0.25) (layer "F.Cu") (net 4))
 (segment (start 151.13 120.65) (end 142.890798 128.889202) (width 0.25) (layer "F.Cu") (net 4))
 (segment (start 149.86 81.28) (end 144.78 86.36) (width 0.25) (layer "F.Cu") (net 4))
 (segment (start 151.13 114.3) (end 151.13 120.65) (width 0.25) (layer "F.Cu") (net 4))
 (segment (start 144.78 86.36) (end 144.78 92.71) (width 0.25) (layer "F.Cu") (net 4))
 (segment (start 172.522499 74.739999) (end 184.1825 86.4) (width 0.25) (layer "F.Cu") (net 4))
 (segment (start 166.37 69.85) (end 171.259999 74.739999) (width 0.25) (layer "F.Cu") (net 4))
 (segment (start 166.37 69.85) (end 154.94 81.28) (width 0.25) (layer "F.Cu") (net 4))
 (segment (start 154.94 81.28) (end 149.86 81.28) (width 0.25) (layer "F.Cu") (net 4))
 (segment (start 150.510799 53.990799) (end 132.772311 53.990799) (width 0.25) (layer "B.Cu") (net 4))
 (segment (start 166.37 69.85) (end 150.510799 53.990799) (width 0.25) (layer "B.Cu") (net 4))
 (segment (start 138.43 126.633759) (end 138.43 114.3) (width 0.4) (layer "B.Cu") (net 4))
 (segment (start 138.43 99.06) (end 138.43 114.3) (width 0.25) (layer "B.Cu") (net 4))
 (segment (start 138.43 99.06) (end 117.075 99.06) (width 0.25) (layer "B.Cu") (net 4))
 (segment (start 117.075 99.06) (end 113.265 95.25) (width 0.25) (layer "B.Cu") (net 4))
 (segment (start 136.174557 128.889202) (end 138.43 126.633759) (width 0.4) (layer "B.Cu") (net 4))
 (segment (start 180.34 60.96) (end 175.26 66.04) (width 0.25) (layer "B.Cu") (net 1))
 (segment (start 175.26 79.328124) (end 167.545 87.043124) (width 0.25) (layer "B.Cu") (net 1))
 (segment (start 167.545 87.043124) (end 167.545 94.075) (width 0.25) (layer "B.Cu") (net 1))
 (segment (start 190.5 66.04) (end 185.42 60.96) (width 0.25) (layer "B.Cu") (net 1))
 (segment (start 175.26 66.04) (end 175.26 79.328124) (width 0.25) (layer "B.Cu") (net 1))
 (segment (start 144.78 111.76) (end 144.78 113.03) (width 0.25) (layer "B.Cu") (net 1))
 (segment (start 152.4 109.22) (end 147.32 109.22) (width 0.25) (layer "B.Cu") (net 1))
 (segment (start 167.545 94.075) (end 152.4 109.22) (width 0.25) (layer "B.Cu") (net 1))
 (segment (start 185.42 60.96) (end 180.34 60.96) (width 0.25) (layer "B.Cu") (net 1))
 (segment (start 144.78 113.03) (end 146.05 114.3) (width 0.25) (layer "B.Cu") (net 1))
 (segment (start 147.32 109.22) (end 144.78 111.76) (width 0.25) (layer "B.Cu") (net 1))
 (segment (start 185.42 66.04) (end 185.42 73.66) (width 0.25) (layer "B.Cu") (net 2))
 (segment (start 175.26 93.98) (end 169.590309 93.98) (width 0.25) (layer "B.Cu") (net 2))
 (segment (start 149.270309 114.3) (end 147.365 114.3) (width 0.25) (layer "B.Cu") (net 2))
 (segment (start 177.8 81.28) (end 175.26 83.82) (width 0.25) (layer "B.Cu") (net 2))
 (segment (start 169.590309 93.98) (end 149.270309 114.3) (width 0.25) (layer "B.Cu") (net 2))
 (segment (start 185.42 73.66) (end 177.8 81.28) (width 0.25) (layer "B.Cu") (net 2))
 (segment (start 175.26 83.82) (end 175.26 93.98) (width 0.25) (layer "B.Cu") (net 2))
 (segment (start 143.51 118.11) (end 143.51 114.3) (width 0.25) (layer "B.Cu") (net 9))
 (segment (start 144.78 119.38) (end 143.51 118.11) (width 0.25) (layer "B.Cu") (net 9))
 (segment (start 184.1575 119.38) (end 187.935 115.6025) (width 0.25) (layer "B.Cu") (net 9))
 (segment (start 184.1575 119.38) (end 144.78 119.38) (width 0.25) (layer "B.Cu") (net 9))
 (segment (start 187.935 115.6025) (end 188 115.6025) (width 0.25) (layer "B.Cu") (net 9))
 (segment (start 140.97 114.3) (end 140.97 120.65) (width 0.25) (layer "B.Cu") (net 10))
 (segment (start 140.97 120.65) (end 147.32 127) (width 0.25) (layer "B.Cu") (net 10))
 (segment (start 190.46 119.42) (end 190.46 115.6025) (width 0.25) (layer "B.Cu") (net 10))
 (segment (start 182.88 127) (end 190.46 119.42) (width 0.25) (layer "B.Cu") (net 10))
 (segment (start 147.32 127) (end 182.88 127) (width 0.25) (layer "B.Cu") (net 10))
 (segment (start 116.84 68.58) (end 121.92 63.5) (width 0.4) (layer "B.Cu") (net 12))
 (segment (start 156.21 67.31) (end 156.21 69.85) (width 0.4) (layer "B.Cu") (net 12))
 (segment (start 152.4 63.5) (end 156.21 67.31) (width 0.4) (layer "B.Cu") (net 12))
 (segment (start 116.84 86.595) (end 116.84 68.58) (width 0.4) (layer "B.Cu") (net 12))
 (segment (start 113.265 90.17) (end 116.84 86.595) (width 0.4) (layer "B.Cu") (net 12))
 (segment (start 121.92 63.5) (end 152.4 63.5) (width 0.4) (layer "B.Cu") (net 12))
 (segment (start 115.57 92.71) (end 134.62 73.66) (width 0.4) (layer "B.Cu") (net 11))
 (segment (start 113.265 92.71) (end 115.57 92.71) (width 0.4) (layer "B.Cu") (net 11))
 (segment (start 154.94 73.66) (end 158.75 69.85) (width 0.4) (layer "B.Cu") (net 11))
 (segment (start 134.62 73.66) (end 154.94 73.66) (width 0.4) (layer "B.Cu") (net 11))
 (segment (start 156.55 55.88) (end 132.08 55.88) (width 0.25) (layer "F.Cu") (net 7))
 (segment (start 131.429201 56.530799) (end 128.372902 56.530799) (width 0.25) (layer "F.Cu") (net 7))
 (segment (start 168.91 68.24) (end 156.55 55.88) (width 0.25) (layer "F.Cu") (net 7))
 (segment (start 132.08 55.88) (end 131.429201 56.530799) (width 0.25) (layer "F.Cu") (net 7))
 (segment (start 168.91 69.85) (end 168.91 68.24) (width 0.25) (layer "F.Cu") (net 7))
 (segment (start 171.45 69.85) (end 172.72 68.58) (width 0.25) (layer "B.Cu") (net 8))
 (segment (start 157.48 48.26) (end 132.08 48.26) (width 0.25) (layer "B.Cu") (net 8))
 (segment (start 172.72 68.58) (end 172.72 63.5) (width 0.25) (layer "B.Cu") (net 8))
 (segment (start 132.08 48.26) (end 130.572606 49.767394) (width 0.25) (layer "B.Cu") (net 8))
 (segment (start 130.572606 49.767394) (end 130.572606 55.260799) (width 0.25) (layer "B.Cu") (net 8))
 (segment (start 172.72 63.5) (end 157.48 48.26) (width 0.25) (layer "B.Cu") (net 8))
 (segment (start 129.54 60.96) (end 129.54 119.38) (width 0.25) (layer "F.Cu") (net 5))
 (segment (start 161.29 69.85) (end 161.29 68.24) (width 0.25) (layer "F.Cu") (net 5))
 (segment (start 132.08 58.42) (end 152.4 58.42) (width 0.25) (layer "F.Cu") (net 5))
 (segment (start 129.54 60.96) (end 132.08 58.42) (width 0.25) (layer "F.Cu") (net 5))
 (segment (start 154.01 60.03) (end 154.01 60.96) (width 0.25) (layer "F.Cu") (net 5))
 (segment (start 161.29 68.24) (end 154.01 60.96) (width 0.25) (layer "F.Cu") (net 5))
 (segment (start 152.4 58.42) (end 154.01 60.03) (width 0.25) (layer "F.Cu") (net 5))
 (segment (start 131.775148 121.615148) (end 131.775148 126.349202) (width 0.25) (layer "F.Cu") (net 5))
 (segment (start 129.54 119.38) (end 131.775148 121.615148) (width 0.25) (layer "F.Cu") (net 5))
 (segment (start 134.62 124.46) (end 133.974852 125.105148) (width 0.25) (layer "F.Cu") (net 6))
 (segment (start 132.08 119.38) (end 134.62 121.92) (width 0.25) (layer "F.Cu") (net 6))
 (segment (start 132.08 81.28) (end 132.08 119.38) (width 0.25) (layer "F.Cu") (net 6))
 (segment (start 133.974852 125.105148) (end 133.974852 127.619202) (width 0.25) (layer "F.Cu") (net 6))
 (segment (start 137.16 76.2) (end 132.08 81.28) (width 0.25) (layer "F.Cu") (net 6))
 (segment (start 134.62 121.92) (end 134.62 124.46) (width 0.25) (layer "F.Cu") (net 6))
 (segment (start 157.48 76.2) (end 137.16 76.2) (width 0.25) (layer "F.Cu") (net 6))
 (segment (start 163.83 69.85) (end 157.48 76.2) (width 0.25) (layer "F.Cu") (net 6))
 (segment (start 143.51 99.06) (end 140.97 96.52) (width 0.4) (layer "B.Cu") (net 26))
 (segment (start 121.92 88.9) (end 123.19 87.63) (width 0.4) (layer "B.Cu") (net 26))
 (segment (start 121.92 93.98) (end 124.46 96.52) (width 0.4) (layer "B.Cu") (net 26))
 (segment (start 121.92 88.9) (end 121.92 93.98) (width 0.4) (layer "B.Cu") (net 26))
 (segment (start 140.97 96.52) (end 124.46 96.52) (width 0.4) (layer "B.Cu") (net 26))
 (segment (start 146.05 99.06) (end 140.97 93.98) (width 0.4) (layer "B.Cu") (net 27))
 (segment (start 124.46 91.44) (end 124.46 88.9) (width 0.4) (layer "B.Cu") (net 27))
 (segment (start 127 93.98) (end 124.46 91.44) (width 0.4) (layer "B.Cu") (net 27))
 (segment (start 140.97 93.98) (end 127 93.98) (width 0.4) (layer "B.Cu") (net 27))
 (segment (start 124.46 88.9) (end 125.73 87.63) (width 0.4) (layer "B.Cu") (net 27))
 (segment (start 137.16 91.44) (end 133.35 87.63) (width 0.4) (layer "B.Cu") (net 30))
 (segment (start 149.86 91.44) (end 137.16 91.44) (width 0.4) (layer "B.Cu") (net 30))
 (segment (start 153.67 99.06) (end 153.67 95.25) (width 0.4) (layer "B.Cu") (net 30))
 (segment (start 153.67 95.25) (end 149.86 91.44) (width 0.4) (layer "B.Cu") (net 30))
 (segment (start 153.67 101.6) (end 157.48 101.6) (width 0.4) (layer "B.Cu") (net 31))
 (segment (start 151.627767 78.74) (end 144.78 78.74) (width 0.4) (layer "B.Cu") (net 31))
 (segment (start 151.13 99.06) (end 153.67 101.6) (width 0.4) (layer "B.Cu") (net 31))
 (segment (start 160.02 99.06) (end 160.02 87.132233) (width 0.4) (layer "B.Cu") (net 31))
 (segment (start 157.48 101.6) (end 160.02 99.06) (width 0.4) (layer "B.Cu") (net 31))
 (segment (start 160.02 87.132233) (end 151.627767 78.74) (width 0.4) (layer "B.Cu") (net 31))
 (segment (start 144.78 78.74) (end 135.89 87.63) (width 0.4) (layer "B.Cu") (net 31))
 (segment (start 139.7 104.14) (end 140.97 102.87) (width 0.25) (layer "F.Cu") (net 32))
 (segment (start 134.62 96.52) (end 134.62 101.6) (width 0.25) (layer "F.Cu") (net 32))
 (segment (start 134.62 101.6) (end 137.16 104.14) (width 0.25) (layer "F.Cu") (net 32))
 (segment (start 138.43 92.71) (end 134.62 96.52) (width 0.25) (layer "F.Cu") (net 32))
 (segment (start 137.16 104.14) (end 139.7 104.14) (width 0.25) (layer "F.Cu") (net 32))
 (segment (start 140.97 102.87) (end 140.97 99.06) (width 0.25) (layer "F.Cu") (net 32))
 (segment (start 138.43 87.63) (end 138.43 92.71) (width 0.25) (layer "F.Cu") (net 32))
 (segment (start 156.21 99.06) (end 156.21 95.25) (width 0.25) (layer "B.Cu") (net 34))
 (segment (start 152.4 91.44) (end 152.4 85.529149) (width 0.25) (layer "B.Cu") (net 34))
 (segment (start 152.4 85.529149) (end 150.690851 83.82) (width 0.25) (layer "B.Cu") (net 34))
 (segment (start 147.32 83.82) (end 143.51 87.63) (width 0.25) (layer "B.Cu") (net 34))
 (segment (start 156.21 95.25) (end 152.4 91.44) (width 0.25) (layer "B.Cu") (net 34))
 (segment (start 150.690851 83.82) (end 147.32 83.82) (width 0.25) (layer "B.Cu") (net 34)))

